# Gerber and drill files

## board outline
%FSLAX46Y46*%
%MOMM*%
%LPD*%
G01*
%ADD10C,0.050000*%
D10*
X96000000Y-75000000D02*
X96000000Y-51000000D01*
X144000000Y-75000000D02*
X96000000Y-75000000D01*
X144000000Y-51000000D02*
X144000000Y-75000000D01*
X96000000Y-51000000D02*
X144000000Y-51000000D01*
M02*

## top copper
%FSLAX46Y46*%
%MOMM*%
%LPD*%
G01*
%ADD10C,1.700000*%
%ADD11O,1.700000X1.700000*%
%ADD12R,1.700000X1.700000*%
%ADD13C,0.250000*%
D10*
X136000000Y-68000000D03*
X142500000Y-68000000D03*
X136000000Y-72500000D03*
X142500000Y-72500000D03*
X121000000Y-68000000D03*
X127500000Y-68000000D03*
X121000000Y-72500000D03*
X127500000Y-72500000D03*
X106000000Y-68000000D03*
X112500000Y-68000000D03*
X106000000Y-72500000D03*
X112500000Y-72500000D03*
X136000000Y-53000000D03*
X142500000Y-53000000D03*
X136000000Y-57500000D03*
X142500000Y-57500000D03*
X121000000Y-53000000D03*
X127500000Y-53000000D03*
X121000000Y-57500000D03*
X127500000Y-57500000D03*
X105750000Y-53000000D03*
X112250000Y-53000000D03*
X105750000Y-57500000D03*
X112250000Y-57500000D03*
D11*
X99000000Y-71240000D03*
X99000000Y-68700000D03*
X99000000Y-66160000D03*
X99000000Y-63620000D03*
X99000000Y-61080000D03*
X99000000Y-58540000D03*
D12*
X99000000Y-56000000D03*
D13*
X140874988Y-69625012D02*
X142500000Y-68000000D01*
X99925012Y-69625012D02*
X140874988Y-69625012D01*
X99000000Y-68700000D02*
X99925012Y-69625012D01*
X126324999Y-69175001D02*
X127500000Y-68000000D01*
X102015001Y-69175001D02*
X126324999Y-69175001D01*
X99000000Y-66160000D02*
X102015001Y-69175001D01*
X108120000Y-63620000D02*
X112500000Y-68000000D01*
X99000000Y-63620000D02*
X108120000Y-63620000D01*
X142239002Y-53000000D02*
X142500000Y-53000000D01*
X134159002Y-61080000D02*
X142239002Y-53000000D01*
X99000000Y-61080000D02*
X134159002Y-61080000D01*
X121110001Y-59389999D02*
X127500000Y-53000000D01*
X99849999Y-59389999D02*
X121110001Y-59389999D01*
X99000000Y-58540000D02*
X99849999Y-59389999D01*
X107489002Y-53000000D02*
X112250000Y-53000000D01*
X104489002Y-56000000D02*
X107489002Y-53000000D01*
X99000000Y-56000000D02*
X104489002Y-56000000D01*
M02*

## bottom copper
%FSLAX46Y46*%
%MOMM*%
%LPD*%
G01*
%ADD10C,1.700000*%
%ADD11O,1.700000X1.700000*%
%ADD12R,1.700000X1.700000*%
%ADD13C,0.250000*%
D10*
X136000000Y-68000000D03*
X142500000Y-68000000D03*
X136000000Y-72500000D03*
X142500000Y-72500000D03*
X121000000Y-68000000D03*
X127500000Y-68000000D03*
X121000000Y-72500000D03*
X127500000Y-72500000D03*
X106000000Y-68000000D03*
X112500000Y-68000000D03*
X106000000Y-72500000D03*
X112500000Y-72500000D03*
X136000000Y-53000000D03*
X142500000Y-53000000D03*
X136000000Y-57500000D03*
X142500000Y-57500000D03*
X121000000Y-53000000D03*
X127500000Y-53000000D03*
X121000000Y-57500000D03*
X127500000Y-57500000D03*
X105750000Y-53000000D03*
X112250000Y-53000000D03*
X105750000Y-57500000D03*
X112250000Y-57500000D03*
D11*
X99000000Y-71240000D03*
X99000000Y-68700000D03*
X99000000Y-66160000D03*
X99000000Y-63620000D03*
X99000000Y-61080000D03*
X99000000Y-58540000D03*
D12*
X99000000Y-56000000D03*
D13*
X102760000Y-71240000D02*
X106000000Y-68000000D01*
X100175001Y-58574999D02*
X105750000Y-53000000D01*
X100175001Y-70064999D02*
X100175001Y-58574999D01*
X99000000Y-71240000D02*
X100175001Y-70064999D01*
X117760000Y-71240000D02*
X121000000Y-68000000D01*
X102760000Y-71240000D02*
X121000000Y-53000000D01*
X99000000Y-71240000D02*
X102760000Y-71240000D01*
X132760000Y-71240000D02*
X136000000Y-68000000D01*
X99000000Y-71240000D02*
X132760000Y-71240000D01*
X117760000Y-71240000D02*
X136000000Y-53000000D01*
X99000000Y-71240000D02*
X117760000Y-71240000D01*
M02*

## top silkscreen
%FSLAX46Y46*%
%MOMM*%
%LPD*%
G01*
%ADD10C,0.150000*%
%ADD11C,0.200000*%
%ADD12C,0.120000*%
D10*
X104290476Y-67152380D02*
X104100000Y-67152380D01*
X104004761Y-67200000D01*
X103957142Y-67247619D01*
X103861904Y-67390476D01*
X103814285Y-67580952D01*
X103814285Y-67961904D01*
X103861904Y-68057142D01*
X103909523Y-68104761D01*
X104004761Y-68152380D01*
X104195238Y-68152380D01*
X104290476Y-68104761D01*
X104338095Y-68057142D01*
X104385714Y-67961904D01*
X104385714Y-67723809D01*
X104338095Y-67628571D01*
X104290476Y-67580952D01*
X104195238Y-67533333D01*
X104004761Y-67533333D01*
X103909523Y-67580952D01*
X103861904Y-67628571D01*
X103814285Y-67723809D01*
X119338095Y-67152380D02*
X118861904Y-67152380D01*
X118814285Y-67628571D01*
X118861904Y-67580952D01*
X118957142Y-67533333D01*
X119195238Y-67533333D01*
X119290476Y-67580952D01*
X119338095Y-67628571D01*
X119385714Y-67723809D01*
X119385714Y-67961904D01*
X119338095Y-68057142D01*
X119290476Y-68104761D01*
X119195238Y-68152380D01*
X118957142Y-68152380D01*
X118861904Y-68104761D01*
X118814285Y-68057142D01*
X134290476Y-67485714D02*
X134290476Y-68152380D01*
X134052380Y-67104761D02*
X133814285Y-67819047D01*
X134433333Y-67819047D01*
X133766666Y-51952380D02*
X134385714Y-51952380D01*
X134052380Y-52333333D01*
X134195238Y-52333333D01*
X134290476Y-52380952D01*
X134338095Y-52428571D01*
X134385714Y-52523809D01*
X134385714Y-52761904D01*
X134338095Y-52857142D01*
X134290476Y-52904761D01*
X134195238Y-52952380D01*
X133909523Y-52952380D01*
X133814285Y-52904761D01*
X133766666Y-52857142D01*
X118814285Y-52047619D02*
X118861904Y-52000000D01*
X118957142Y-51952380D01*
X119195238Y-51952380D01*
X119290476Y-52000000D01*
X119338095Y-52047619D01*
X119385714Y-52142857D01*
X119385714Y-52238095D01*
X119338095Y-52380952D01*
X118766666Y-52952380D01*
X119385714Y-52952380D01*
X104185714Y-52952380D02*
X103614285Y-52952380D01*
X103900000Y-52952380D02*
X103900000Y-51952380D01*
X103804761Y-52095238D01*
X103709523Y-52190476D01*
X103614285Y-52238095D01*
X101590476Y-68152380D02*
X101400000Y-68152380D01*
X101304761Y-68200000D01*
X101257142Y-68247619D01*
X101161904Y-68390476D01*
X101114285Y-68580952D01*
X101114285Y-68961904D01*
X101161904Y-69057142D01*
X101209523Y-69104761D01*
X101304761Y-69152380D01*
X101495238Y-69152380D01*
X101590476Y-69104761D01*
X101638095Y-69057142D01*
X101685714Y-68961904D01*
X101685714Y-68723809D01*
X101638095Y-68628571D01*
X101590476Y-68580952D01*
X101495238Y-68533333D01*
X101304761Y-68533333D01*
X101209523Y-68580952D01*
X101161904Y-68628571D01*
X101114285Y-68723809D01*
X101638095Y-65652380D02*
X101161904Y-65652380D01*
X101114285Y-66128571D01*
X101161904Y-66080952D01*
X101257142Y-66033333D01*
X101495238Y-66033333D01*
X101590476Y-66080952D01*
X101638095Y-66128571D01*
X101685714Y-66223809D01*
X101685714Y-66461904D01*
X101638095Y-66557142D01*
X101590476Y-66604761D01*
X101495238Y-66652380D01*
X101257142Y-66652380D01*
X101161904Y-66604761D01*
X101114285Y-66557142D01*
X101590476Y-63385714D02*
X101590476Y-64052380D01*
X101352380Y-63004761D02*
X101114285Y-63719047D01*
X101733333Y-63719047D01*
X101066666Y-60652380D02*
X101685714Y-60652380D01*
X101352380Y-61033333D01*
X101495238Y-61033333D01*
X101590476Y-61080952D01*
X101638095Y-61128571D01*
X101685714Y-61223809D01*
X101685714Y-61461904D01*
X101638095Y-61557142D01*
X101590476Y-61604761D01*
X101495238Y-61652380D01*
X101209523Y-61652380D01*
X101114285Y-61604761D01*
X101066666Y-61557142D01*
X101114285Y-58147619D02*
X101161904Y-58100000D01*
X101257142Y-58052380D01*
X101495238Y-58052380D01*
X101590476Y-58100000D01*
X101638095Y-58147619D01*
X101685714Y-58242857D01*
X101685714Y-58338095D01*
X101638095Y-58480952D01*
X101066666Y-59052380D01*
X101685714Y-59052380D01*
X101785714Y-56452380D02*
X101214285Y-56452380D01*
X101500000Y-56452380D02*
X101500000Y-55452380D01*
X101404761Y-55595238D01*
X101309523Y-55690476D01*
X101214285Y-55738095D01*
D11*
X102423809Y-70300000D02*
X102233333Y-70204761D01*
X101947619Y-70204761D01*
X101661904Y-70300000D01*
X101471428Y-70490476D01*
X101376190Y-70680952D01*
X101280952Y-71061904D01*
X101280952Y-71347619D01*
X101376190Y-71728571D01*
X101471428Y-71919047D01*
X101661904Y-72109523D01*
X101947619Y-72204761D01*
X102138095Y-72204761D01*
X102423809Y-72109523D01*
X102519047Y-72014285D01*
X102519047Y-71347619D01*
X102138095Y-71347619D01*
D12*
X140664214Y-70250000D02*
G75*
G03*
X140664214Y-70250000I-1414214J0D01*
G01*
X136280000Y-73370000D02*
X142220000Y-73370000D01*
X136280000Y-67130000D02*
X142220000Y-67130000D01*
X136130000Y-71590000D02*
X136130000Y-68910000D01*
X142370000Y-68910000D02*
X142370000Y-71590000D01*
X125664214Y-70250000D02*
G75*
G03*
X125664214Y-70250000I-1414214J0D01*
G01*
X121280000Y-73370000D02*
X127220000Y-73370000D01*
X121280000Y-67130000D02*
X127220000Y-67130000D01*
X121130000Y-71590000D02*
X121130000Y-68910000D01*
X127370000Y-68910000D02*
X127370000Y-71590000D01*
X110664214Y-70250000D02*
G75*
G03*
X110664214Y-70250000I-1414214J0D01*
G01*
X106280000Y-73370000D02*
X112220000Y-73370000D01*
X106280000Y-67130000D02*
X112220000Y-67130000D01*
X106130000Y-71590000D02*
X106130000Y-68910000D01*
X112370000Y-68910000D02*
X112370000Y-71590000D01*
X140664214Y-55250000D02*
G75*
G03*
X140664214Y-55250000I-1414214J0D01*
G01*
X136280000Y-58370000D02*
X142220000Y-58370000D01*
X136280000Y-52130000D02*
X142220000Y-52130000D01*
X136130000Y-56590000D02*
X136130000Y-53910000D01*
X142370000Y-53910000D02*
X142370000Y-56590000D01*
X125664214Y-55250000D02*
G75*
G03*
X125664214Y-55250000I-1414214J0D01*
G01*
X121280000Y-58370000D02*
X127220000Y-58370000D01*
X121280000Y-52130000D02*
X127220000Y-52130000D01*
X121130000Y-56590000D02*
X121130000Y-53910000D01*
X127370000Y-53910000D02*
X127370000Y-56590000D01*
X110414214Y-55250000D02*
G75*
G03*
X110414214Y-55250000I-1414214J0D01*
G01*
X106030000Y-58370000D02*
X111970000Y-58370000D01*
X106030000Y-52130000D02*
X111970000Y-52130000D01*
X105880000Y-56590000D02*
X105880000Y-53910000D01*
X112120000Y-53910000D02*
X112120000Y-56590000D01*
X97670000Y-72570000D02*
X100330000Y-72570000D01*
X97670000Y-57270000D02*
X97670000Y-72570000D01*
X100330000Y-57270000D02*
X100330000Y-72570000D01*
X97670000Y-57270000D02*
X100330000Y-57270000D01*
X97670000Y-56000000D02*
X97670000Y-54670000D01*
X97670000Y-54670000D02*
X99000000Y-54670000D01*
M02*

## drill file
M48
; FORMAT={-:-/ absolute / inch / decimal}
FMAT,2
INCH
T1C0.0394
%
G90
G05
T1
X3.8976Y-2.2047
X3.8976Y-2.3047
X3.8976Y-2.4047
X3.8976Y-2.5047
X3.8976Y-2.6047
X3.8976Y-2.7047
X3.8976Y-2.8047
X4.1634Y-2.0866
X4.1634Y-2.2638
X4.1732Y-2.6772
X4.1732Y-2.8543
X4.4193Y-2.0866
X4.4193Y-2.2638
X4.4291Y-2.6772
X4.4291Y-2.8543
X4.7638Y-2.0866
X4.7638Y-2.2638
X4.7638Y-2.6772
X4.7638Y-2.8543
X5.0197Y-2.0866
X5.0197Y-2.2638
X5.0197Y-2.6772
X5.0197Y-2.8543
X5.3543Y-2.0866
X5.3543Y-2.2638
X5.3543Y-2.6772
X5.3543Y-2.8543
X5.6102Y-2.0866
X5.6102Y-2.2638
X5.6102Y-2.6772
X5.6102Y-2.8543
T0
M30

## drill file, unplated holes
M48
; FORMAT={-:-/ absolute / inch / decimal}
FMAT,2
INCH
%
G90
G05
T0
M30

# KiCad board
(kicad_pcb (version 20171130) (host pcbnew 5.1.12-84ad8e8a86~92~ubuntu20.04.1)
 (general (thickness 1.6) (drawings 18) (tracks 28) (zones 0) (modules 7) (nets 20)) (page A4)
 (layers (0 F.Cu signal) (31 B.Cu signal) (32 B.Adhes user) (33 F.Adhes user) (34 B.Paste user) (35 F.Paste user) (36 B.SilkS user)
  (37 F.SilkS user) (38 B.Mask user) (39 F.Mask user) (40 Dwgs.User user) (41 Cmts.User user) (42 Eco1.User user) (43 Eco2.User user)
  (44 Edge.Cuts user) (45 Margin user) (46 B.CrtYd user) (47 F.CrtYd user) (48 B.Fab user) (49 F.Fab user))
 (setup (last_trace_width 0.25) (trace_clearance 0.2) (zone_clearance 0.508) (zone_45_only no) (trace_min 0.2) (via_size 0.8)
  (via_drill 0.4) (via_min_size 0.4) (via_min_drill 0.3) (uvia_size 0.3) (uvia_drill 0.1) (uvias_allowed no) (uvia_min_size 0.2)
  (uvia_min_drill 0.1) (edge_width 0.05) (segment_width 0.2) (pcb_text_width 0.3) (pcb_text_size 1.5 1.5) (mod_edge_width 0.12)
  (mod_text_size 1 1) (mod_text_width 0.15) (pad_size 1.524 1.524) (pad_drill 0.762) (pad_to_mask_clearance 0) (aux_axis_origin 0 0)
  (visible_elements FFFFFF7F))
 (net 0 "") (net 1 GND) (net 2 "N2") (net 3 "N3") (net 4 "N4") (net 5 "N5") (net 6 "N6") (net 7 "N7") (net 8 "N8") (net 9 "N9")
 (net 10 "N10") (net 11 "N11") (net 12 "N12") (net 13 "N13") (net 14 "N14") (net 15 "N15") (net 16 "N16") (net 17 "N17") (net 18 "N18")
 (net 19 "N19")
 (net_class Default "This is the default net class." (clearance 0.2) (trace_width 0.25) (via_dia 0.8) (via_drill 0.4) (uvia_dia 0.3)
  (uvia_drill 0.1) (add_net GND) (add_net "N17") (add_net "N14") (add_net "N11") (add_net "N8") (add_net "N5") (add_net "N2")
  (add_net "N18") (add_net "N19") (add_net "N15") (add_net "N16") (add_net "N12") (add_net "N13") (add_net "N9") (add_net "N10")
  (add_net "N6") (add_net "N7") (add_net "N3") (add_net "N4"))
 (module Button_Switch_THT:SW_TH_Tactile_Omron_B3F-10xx (layer F.Cu) (at 136 68)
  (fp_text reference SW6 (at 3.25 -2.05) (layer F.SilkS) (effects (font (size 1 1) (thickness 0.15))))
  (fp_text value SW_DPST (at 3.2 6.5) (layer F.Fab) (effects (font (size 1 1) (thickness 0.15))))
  (fp_circle (center 3.25 2.25) (end 4.25 3.25) (layer F.SilkS) (width 0.12))
  (fp_line (start 0.28 5.37) (end 6.22 5.37) (layer F.SilkS) (width 0.12))
  (fp_line (start 0.28 -0.87) (end 6.22 -0.87) (layer F.SilkS) (width 0.12))
  (fp_line (start 0.13 3.59) (end 0.13 0.91) (layer F.SilkS) (width 0.12))
  (fp_line (start 6.37 0.91) (end 6.37 3.59) (layer F.SilkS) (width 0.12))
  (pad 1 thru_hole circle (at 0 0) (size 1.7 1.7) (drill 1) (layers *.Cu *.Mask) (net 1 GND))
  (pad 2 thru_hole circle (at 6.5 0) (size 1.7 1.7) (drill 1) (layers *.Cu *.Mask) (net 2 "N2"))
  (pad 3 thru_hole circle (at 0 4.5) (size 1.7 1.7) (drill 1) (layers *.Cu *.Mask) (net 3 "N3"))
  (pad 4 thru_hole circle (at 6.5 4.5) (size 1.7 1.7) (drill 1) (layers *.Cu *.Mask) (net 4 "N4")))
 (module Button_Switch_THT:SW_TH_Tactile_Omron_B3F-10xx (layer F.Cu) (at 121 68)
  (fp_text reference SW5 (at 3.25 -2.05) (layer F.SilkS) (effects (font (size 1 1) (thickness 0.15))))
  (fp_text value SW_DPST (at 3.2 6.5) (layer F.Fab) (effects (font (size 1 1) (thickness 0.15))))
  (fp_circle (center 3.25 2.25) (end 4.25 3.25) (layer F.SilkS) (width 0.12))
  (fp_line (start 0.28 5.37) (end 6.22 5.37) (layer F.SilkS) (width 0.12))
  (fp_line (start 0.28 -0.87) (end 6.22 -0.87) (layer F.SilkS) (width 0.12))
  (fp_line (start 0.13 3.59) (end 0.13 0.91) (layer F.SilkS) (width 0.12))
  (fp_line (start 6.37 0.91) (end 6.37 3.59) (layer F.SilkS) (width 0.12))
  (pad 1 thru_hole circle (at 0 0) (size 1.7 1.7) (drill 1) (layers *.Cu *.Mask) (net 1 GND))
  (pad 2 thru_hole circle (at 6.5 0) (size 1.7 1.7) (drill 1) (layers *.Cu *.Mask) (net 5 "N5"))
  (pad 3 thru_hole circle (at 0 4.5) (size 1.7 1.7) (drill 1) (layers *.Cu *.Mask) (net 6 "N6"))
  (pad 4 thru_hole circle (at 6.5 4.5) (size 1.7 1.7) (drill 1) (layers *.Cu *.Mask) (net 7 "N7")))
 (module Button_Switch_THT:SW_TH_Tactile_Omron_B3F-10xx (layer F.Cu) (at 106 68)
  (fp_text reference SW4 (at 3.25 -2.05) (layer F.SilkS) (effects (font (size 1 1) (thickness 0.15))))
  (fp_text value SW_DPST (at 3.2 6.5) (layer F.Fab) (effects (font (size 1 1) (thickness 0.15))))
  (fp_circle (center 3.25 2.25) (end 4.25 3.25) (layer F.SilkS) (width 0.12))
  (fp_line (start 0.28 5.37) (end 6.22 5.37) (layer F.SilkS) (width 0.12))
  (fp_line (start 0.28 -0.87) (end 6.22 -0.87) (layer F.SilkS) (width 0.12))
  (fp_line (start 0.13 3.59) (end 0.13 0.91) (layer F.SilkS) (width 0.12))
  (fp_line (start 6.37 0.91) (end 6.37 3.59) (layer F.SilkS) (width 0.12))
  (pad 1 thru_hole circle (at 0 0) (size 1.7 1.7) (drill 1) (layers *.Cu *.Mask) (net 1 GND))
  (pad 2 thru_hole circle (at 6.5 0) (size 1.7 1.7) (drill 1) (layers *.Cu *.Mask) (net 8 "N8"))
  (pad 3 thru_hole circle (at 0 4.5) (size 1.7 1.7) (drill 1) (layers *.Cu *.Mask) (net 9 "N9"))
  (pad 4 thru_hole circle (at 6.5 4.5) (size 1.7 1.7) (drill 1) (layers *.Cu *.Mask) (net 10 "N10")))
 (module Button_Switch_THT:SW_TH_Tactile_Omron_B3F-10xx (layer F.Cu) (at 136 53)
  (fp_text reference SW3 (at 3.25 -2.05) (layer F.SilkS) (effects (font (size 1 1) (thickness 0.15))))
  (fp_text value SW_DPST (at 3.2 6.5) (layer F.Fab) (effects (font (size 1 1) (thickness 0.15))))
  (fp_circle (center 3.25 2.25) (end 4.25 3.25) (layer F.SilkS) (width 0.12))
  (fp_line (start 0.28 5.37) (end 6.22 5.37) (layer F.SilkS) (width 0.12))
  (fp_line (start 0.28 -0.87) (end 6.22 -0.87) (layer F.SilkS) (width 0.12))
  (fp_line (start 0.13 3.59) (end 0.13 0.91) (layer F.SilkS) (width 0.12))
  (fp_line (start 6.37 0.91) (end 6.37 3.59) (layer F.SilkS) (width 0.12))
  (pad 1 thru_hole circle (at 0 0) (size 1.7 1.7) (drill 1) (layers *.Cu *.Mask) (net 1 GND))
  (pad 2 thru_hole circle (at 6.5 0) (size 1.7 1.7) (drill 1) (layers *.Cu *.Mask) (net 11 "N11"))
  (pad 3 thru_hole circle (at 0 4.5) (size 1.7 1.7) (drill 1) (layers *.Cu *.Mask) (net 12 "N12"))
  (pad 4 thru_hole circle (at 6.5 4.5) (size 1.7 1.7) (drill 1) (layers *.Cu *.Mask) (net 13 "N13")))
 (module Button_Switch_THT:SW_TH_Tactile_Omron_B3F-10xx (layer F.Cu) (at 121 53)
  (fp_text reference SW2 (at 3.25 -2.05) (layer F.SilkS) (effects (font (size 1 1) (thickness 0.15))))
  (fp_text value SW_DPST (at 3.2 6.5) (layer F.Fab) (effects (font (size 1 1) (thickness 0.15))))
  (fp_circle (center 3.25 2.25) (end 4.25 3.25) (layer F.SilkS) (width 0.12))
  (fp_line (start 0.28 5.37) (end 6.22 5.37) (layer F.SilkS) (width 0.12))
  (fp_line (start 0.28 -0.87) (end 6.22 -0.87) (layer F.SilkS) (width 0.12))
  (fp_line (start 0.13 3.59) (end 0.13 0.91) (layer F.SilkS) (width 0.12))
  (fp_line (start 6.37 0.91) (end 6.37 3.59) (layer F.SilkS) (width 0.12))
  (pad 1 thru_hole circle (at 0 0) (size 1.7 1.7) (drill 1) (layers *.Cu *.Mask) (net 1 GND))
  (pad 2 thru_hole circle (at 6.5 0) (size 1.7 1.7) (drill 1) (layers *.Cu *.Mask) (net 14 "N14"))
  (pad 3 thru_hole circle (at 0 4.5) (size 1.7 1.7) (drill 1) (layers *.Cu *.Mask) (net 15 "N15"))
  (pad 4 thru_hole circle (at 6.5 4.5) (size 1.7 1.7) (drill 1) (layers *.Cu *.Mask) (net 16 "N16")))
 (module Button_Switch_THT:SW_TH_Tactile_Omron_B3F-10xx (layer F.Cu) (at 105.75 53)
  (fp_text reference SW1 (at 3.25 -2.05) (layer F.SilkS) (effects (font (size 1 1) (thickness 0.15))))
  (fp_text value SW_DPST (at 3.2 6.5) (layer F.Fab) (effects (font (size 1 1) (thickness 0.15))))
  (fp_circle (center 3.25 2.25) (end 4.25 3.25) (layer F.SilkS) (width 0.12))
  (fp_line (start 0.28 5.37) (end 6.22 5.37) (layer F.SilkS) (width 0.12))
  (fp_line (start 0.28 -0.87) (end 6.22 -0.87) (layer F.SilkS) (width 0.12))
  (fp_line (start 0.13 3.59) (end 0.13 0.91) (layer F.SilkS) (width 0.12))
  (fp_line (start 6.37 0.91) (end 6.37 3.59) (layer F.SilkS) (width 0.12))
  (pad 1 thru_hole circle (at 0 0) (size 1.7 1.7) (drill 1) (layers *.Cu *.Mask) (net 1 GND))
  (pad 2 thru_hole circle (at 6.5 0) (size 1.7 1.7) (drill 1) (layers *.Cu *.Mask) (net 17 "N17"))
  (pad 3 thru_hole circle (at 0 4.5) (size 1.7 1.7) (drill 1) (layers *.Cu *.Mask) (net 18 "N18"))
  (pad 4 thru_hole circle (at 6.5 4.5) (size 1.7 1.7) (drill 1) (layers *.Cu *.Mask) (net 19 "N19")))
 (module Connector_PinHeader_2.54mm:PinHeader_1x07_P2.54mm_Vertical (layer F.Cu) (at 99 56)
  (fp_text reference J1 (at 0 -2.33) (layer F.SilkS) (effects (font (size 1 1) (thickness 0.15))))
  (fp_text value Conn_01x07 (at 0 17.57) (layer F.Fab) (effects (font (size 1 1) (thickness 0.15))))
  (fp_line (start -1.33 16.57) (end 1.33 16.57) (layer F.SilkS) (width 0.12))
  (fp_line (start -1.33 1.27) (end -1.33 16.57) (layer F.SilkS) (width 0.12))
  (fp_line (start 1.33 1.27) (end 1.33 16.57) (layer F.SilkS) (width 0.12))
  (fp_line (start -1.33 1.27) (end 1.33 1.27) (layer F.SilkS) (width 0.12))
  (fp_line (start -1.33 0) (end -1.33 -1.33) (layer F.SilkS) (width 0.12))
  (fp_line (start -1.33 -1.33) (end 0 -1.33) (layer F.SilkS) (width 0.12))
  (pad 7 thru_hole oval (at 0 15.24) (size 1.7 1.7) (drill 1) (layers *.Cu *.Mask) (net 1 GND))
  (pad 6 thru_hole oval (at 0 12.7) (size 1.7 1.7) (drill 1) (layers *.Cu *.Mask) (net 2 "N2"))
  (pad 5 thru_hole oval (at 0 10.16) (size 1.7 1.7) (drill 1) (layers *.Cu *.Mask) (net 5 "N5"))
  (pad 4 thru_hole oval (at 0 7.62) (size 1.7 1.7) (drill 1) (layers *.Cu *.Mask) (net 8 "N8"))
  (pad 3 thru_hole oval (at 0 5.08) (size 1.7 1.7) (drill 1) (layers *.Cu *.Mask) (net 11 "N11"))
  (pad 2 thru_hole oval (at 0 2.54) (size 1.7 1.7) (drill 1) (layers *.Cu *.Mask) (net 14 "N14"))
  (pad 1 thru_hole rect (at 0 0) (size 1.7 1.7) (drill 1) (layers *.Cu *.Mask) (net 17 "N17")))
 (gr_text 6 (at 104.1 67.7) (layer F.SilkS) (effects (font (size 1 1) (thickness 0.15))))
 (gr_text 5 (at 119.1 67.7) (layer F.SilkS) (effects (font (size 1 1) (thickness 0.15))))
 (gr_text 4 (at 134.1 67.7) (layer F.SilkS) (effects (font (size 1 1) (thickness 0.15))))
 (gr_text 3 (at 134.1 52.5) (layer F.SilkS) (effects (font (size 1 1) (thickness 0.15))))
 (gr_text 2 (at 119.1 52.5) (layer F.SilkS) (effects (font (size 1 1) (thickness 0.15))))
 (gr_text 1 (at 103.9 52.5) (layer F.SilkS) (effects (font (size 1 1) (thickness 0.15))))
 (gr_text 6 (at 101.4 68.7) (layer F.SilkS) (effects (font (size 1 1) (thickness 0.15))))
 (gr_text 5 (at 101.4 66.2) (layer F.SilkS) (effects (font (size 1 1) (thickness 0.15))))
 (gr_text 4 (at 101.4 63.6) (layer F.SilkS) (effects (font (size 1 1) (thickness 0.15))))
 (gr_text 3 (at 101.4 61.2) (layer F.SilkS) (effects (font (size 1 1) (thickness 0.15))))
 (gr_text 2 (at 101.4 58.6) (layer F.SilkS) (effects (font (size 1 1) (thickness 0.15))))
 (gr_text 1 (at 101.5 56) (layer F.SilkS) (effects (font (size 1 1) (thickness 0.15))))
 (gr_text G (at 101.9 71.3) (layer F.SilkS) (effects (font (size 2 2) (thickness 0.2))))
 (gr_line (start 96 75) (end 96 51) (layer Edge.Cuts) (width 0.05))
 (gr_line (start 144 75) (end 96 75) (layer Edge.Cuts) (width 0.05))
 (gr_line (start 144 51) (end 144 75) (layer Edge.Cuts) (width 0.05))
 (gr_line (start 96 51) (end 144 51) (layer Edge.Cuts) (width 0.05))
 (segment (start 102.76 71.24) (end 106 68) (width 0.25) (layer B.Cu) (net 1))
 (segment (start 100.175001 58.574999) (end 105.75 53) (width 0.25) (layer B.Cu) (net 1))
 (segment (start 100.175001 70.064999) (end 100.175001 58.574999) (width 0.25) (layer B.Cu) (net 1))
 (segment (start 99 71.24) (end 100.175001 70.064999) (width 0.25) (layer B.Cu) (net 1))
 (segment (start 117.76 71.24) (end 121 68) (width 0.25) (layer B.Cu) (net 1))
 (segment (start 102.76 71.24) (end 121 53) (width 0.25) (layer B.Cu) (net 1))
 (segment (start 99 71.24) (end 102.76 71.24) (width 0.25) (layer B.Cu) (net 1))
 (segment (start 132.76 71.24) (end 136 68) (width 0.25) (layer B.Cu) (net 1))
 (segment (start 99 71.24) (end 132.76 71.24) (width 0.25) (layer B.Cu) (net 1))
 (segment (start 117.76 71.24) (end 136 53) (width 0.25) (layer B.Cu) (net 1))
 (segment (start 99 71.24) (end 117.76 71.24) (width 0.25) (layer B.Cu) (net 1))
 (segment (start 140.874988 69.625012) (end 142.5 68) (width 0.25) (layer F.Cu) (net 2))
 (segment (start 99.925012 69.625012) (end 140.874988 69.625012) (width 0.25) (layer F.Cu) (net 2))
 (segment (start 99 68.7) (end 99.925012 69.625012) (width 0.25) (layer F.Cu) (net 2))
 (segment (start 126.324999 69.175001) (end 127.5 68) (width 0.25) (layer F.Cu) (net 5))
 (segment (start 102.015001 69.175001) (end 126.324999 69.175001) (width 0.25) (layer F.Cu) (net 5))
 (segment (start 99 66.16) (end 102.015001 69.175001) (width 0.25) (layer F.Cu) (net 5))
 (segment (start 108.12 63.62) (end 112.5 68) (width 0.25) (layer F.Cu) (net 8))
 (segment (start 99 63.62) (end 108.12 63.62) (width 0.25) (layer F.Cu) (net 8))
 (segment (start 142.239002 53) (end 142.5 53) (width 0.25) (layer F.Cu) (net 11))
 (segment (start 134.159002 61.08) (end 142.239002 53) (width 0.25) (layer F.Cu) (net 11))
 (segment (start 99 61.08) (end 134.159002 61.08) (width 0.25) (layer F.Cu) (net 11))
 (segment (start 121.110001 59.389999) (end 127.5 53) (width 0.25) (layer F.Cu) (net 14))
 (segment (start 99.849999 59.389999) (end 121.110001 59.389999) (width 0.25) (layer F.Cu) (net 14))
 (segment (start 99 58.54) (end 99.849999 59.389999) (width 0.25) (layer F.Cu) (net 14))
 (segment (start 107.489002 53) (end 112.25 53) (width 0.25) (layer F.Cu) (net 17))
 (segment (start 104.489002 56) (end 107.489002 53) (width 0.25) (layer F.Cu) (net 17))
 (segment (start 99 56) (end 104.489002 56) (width 0.25) (layer F.Cu) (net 17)))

